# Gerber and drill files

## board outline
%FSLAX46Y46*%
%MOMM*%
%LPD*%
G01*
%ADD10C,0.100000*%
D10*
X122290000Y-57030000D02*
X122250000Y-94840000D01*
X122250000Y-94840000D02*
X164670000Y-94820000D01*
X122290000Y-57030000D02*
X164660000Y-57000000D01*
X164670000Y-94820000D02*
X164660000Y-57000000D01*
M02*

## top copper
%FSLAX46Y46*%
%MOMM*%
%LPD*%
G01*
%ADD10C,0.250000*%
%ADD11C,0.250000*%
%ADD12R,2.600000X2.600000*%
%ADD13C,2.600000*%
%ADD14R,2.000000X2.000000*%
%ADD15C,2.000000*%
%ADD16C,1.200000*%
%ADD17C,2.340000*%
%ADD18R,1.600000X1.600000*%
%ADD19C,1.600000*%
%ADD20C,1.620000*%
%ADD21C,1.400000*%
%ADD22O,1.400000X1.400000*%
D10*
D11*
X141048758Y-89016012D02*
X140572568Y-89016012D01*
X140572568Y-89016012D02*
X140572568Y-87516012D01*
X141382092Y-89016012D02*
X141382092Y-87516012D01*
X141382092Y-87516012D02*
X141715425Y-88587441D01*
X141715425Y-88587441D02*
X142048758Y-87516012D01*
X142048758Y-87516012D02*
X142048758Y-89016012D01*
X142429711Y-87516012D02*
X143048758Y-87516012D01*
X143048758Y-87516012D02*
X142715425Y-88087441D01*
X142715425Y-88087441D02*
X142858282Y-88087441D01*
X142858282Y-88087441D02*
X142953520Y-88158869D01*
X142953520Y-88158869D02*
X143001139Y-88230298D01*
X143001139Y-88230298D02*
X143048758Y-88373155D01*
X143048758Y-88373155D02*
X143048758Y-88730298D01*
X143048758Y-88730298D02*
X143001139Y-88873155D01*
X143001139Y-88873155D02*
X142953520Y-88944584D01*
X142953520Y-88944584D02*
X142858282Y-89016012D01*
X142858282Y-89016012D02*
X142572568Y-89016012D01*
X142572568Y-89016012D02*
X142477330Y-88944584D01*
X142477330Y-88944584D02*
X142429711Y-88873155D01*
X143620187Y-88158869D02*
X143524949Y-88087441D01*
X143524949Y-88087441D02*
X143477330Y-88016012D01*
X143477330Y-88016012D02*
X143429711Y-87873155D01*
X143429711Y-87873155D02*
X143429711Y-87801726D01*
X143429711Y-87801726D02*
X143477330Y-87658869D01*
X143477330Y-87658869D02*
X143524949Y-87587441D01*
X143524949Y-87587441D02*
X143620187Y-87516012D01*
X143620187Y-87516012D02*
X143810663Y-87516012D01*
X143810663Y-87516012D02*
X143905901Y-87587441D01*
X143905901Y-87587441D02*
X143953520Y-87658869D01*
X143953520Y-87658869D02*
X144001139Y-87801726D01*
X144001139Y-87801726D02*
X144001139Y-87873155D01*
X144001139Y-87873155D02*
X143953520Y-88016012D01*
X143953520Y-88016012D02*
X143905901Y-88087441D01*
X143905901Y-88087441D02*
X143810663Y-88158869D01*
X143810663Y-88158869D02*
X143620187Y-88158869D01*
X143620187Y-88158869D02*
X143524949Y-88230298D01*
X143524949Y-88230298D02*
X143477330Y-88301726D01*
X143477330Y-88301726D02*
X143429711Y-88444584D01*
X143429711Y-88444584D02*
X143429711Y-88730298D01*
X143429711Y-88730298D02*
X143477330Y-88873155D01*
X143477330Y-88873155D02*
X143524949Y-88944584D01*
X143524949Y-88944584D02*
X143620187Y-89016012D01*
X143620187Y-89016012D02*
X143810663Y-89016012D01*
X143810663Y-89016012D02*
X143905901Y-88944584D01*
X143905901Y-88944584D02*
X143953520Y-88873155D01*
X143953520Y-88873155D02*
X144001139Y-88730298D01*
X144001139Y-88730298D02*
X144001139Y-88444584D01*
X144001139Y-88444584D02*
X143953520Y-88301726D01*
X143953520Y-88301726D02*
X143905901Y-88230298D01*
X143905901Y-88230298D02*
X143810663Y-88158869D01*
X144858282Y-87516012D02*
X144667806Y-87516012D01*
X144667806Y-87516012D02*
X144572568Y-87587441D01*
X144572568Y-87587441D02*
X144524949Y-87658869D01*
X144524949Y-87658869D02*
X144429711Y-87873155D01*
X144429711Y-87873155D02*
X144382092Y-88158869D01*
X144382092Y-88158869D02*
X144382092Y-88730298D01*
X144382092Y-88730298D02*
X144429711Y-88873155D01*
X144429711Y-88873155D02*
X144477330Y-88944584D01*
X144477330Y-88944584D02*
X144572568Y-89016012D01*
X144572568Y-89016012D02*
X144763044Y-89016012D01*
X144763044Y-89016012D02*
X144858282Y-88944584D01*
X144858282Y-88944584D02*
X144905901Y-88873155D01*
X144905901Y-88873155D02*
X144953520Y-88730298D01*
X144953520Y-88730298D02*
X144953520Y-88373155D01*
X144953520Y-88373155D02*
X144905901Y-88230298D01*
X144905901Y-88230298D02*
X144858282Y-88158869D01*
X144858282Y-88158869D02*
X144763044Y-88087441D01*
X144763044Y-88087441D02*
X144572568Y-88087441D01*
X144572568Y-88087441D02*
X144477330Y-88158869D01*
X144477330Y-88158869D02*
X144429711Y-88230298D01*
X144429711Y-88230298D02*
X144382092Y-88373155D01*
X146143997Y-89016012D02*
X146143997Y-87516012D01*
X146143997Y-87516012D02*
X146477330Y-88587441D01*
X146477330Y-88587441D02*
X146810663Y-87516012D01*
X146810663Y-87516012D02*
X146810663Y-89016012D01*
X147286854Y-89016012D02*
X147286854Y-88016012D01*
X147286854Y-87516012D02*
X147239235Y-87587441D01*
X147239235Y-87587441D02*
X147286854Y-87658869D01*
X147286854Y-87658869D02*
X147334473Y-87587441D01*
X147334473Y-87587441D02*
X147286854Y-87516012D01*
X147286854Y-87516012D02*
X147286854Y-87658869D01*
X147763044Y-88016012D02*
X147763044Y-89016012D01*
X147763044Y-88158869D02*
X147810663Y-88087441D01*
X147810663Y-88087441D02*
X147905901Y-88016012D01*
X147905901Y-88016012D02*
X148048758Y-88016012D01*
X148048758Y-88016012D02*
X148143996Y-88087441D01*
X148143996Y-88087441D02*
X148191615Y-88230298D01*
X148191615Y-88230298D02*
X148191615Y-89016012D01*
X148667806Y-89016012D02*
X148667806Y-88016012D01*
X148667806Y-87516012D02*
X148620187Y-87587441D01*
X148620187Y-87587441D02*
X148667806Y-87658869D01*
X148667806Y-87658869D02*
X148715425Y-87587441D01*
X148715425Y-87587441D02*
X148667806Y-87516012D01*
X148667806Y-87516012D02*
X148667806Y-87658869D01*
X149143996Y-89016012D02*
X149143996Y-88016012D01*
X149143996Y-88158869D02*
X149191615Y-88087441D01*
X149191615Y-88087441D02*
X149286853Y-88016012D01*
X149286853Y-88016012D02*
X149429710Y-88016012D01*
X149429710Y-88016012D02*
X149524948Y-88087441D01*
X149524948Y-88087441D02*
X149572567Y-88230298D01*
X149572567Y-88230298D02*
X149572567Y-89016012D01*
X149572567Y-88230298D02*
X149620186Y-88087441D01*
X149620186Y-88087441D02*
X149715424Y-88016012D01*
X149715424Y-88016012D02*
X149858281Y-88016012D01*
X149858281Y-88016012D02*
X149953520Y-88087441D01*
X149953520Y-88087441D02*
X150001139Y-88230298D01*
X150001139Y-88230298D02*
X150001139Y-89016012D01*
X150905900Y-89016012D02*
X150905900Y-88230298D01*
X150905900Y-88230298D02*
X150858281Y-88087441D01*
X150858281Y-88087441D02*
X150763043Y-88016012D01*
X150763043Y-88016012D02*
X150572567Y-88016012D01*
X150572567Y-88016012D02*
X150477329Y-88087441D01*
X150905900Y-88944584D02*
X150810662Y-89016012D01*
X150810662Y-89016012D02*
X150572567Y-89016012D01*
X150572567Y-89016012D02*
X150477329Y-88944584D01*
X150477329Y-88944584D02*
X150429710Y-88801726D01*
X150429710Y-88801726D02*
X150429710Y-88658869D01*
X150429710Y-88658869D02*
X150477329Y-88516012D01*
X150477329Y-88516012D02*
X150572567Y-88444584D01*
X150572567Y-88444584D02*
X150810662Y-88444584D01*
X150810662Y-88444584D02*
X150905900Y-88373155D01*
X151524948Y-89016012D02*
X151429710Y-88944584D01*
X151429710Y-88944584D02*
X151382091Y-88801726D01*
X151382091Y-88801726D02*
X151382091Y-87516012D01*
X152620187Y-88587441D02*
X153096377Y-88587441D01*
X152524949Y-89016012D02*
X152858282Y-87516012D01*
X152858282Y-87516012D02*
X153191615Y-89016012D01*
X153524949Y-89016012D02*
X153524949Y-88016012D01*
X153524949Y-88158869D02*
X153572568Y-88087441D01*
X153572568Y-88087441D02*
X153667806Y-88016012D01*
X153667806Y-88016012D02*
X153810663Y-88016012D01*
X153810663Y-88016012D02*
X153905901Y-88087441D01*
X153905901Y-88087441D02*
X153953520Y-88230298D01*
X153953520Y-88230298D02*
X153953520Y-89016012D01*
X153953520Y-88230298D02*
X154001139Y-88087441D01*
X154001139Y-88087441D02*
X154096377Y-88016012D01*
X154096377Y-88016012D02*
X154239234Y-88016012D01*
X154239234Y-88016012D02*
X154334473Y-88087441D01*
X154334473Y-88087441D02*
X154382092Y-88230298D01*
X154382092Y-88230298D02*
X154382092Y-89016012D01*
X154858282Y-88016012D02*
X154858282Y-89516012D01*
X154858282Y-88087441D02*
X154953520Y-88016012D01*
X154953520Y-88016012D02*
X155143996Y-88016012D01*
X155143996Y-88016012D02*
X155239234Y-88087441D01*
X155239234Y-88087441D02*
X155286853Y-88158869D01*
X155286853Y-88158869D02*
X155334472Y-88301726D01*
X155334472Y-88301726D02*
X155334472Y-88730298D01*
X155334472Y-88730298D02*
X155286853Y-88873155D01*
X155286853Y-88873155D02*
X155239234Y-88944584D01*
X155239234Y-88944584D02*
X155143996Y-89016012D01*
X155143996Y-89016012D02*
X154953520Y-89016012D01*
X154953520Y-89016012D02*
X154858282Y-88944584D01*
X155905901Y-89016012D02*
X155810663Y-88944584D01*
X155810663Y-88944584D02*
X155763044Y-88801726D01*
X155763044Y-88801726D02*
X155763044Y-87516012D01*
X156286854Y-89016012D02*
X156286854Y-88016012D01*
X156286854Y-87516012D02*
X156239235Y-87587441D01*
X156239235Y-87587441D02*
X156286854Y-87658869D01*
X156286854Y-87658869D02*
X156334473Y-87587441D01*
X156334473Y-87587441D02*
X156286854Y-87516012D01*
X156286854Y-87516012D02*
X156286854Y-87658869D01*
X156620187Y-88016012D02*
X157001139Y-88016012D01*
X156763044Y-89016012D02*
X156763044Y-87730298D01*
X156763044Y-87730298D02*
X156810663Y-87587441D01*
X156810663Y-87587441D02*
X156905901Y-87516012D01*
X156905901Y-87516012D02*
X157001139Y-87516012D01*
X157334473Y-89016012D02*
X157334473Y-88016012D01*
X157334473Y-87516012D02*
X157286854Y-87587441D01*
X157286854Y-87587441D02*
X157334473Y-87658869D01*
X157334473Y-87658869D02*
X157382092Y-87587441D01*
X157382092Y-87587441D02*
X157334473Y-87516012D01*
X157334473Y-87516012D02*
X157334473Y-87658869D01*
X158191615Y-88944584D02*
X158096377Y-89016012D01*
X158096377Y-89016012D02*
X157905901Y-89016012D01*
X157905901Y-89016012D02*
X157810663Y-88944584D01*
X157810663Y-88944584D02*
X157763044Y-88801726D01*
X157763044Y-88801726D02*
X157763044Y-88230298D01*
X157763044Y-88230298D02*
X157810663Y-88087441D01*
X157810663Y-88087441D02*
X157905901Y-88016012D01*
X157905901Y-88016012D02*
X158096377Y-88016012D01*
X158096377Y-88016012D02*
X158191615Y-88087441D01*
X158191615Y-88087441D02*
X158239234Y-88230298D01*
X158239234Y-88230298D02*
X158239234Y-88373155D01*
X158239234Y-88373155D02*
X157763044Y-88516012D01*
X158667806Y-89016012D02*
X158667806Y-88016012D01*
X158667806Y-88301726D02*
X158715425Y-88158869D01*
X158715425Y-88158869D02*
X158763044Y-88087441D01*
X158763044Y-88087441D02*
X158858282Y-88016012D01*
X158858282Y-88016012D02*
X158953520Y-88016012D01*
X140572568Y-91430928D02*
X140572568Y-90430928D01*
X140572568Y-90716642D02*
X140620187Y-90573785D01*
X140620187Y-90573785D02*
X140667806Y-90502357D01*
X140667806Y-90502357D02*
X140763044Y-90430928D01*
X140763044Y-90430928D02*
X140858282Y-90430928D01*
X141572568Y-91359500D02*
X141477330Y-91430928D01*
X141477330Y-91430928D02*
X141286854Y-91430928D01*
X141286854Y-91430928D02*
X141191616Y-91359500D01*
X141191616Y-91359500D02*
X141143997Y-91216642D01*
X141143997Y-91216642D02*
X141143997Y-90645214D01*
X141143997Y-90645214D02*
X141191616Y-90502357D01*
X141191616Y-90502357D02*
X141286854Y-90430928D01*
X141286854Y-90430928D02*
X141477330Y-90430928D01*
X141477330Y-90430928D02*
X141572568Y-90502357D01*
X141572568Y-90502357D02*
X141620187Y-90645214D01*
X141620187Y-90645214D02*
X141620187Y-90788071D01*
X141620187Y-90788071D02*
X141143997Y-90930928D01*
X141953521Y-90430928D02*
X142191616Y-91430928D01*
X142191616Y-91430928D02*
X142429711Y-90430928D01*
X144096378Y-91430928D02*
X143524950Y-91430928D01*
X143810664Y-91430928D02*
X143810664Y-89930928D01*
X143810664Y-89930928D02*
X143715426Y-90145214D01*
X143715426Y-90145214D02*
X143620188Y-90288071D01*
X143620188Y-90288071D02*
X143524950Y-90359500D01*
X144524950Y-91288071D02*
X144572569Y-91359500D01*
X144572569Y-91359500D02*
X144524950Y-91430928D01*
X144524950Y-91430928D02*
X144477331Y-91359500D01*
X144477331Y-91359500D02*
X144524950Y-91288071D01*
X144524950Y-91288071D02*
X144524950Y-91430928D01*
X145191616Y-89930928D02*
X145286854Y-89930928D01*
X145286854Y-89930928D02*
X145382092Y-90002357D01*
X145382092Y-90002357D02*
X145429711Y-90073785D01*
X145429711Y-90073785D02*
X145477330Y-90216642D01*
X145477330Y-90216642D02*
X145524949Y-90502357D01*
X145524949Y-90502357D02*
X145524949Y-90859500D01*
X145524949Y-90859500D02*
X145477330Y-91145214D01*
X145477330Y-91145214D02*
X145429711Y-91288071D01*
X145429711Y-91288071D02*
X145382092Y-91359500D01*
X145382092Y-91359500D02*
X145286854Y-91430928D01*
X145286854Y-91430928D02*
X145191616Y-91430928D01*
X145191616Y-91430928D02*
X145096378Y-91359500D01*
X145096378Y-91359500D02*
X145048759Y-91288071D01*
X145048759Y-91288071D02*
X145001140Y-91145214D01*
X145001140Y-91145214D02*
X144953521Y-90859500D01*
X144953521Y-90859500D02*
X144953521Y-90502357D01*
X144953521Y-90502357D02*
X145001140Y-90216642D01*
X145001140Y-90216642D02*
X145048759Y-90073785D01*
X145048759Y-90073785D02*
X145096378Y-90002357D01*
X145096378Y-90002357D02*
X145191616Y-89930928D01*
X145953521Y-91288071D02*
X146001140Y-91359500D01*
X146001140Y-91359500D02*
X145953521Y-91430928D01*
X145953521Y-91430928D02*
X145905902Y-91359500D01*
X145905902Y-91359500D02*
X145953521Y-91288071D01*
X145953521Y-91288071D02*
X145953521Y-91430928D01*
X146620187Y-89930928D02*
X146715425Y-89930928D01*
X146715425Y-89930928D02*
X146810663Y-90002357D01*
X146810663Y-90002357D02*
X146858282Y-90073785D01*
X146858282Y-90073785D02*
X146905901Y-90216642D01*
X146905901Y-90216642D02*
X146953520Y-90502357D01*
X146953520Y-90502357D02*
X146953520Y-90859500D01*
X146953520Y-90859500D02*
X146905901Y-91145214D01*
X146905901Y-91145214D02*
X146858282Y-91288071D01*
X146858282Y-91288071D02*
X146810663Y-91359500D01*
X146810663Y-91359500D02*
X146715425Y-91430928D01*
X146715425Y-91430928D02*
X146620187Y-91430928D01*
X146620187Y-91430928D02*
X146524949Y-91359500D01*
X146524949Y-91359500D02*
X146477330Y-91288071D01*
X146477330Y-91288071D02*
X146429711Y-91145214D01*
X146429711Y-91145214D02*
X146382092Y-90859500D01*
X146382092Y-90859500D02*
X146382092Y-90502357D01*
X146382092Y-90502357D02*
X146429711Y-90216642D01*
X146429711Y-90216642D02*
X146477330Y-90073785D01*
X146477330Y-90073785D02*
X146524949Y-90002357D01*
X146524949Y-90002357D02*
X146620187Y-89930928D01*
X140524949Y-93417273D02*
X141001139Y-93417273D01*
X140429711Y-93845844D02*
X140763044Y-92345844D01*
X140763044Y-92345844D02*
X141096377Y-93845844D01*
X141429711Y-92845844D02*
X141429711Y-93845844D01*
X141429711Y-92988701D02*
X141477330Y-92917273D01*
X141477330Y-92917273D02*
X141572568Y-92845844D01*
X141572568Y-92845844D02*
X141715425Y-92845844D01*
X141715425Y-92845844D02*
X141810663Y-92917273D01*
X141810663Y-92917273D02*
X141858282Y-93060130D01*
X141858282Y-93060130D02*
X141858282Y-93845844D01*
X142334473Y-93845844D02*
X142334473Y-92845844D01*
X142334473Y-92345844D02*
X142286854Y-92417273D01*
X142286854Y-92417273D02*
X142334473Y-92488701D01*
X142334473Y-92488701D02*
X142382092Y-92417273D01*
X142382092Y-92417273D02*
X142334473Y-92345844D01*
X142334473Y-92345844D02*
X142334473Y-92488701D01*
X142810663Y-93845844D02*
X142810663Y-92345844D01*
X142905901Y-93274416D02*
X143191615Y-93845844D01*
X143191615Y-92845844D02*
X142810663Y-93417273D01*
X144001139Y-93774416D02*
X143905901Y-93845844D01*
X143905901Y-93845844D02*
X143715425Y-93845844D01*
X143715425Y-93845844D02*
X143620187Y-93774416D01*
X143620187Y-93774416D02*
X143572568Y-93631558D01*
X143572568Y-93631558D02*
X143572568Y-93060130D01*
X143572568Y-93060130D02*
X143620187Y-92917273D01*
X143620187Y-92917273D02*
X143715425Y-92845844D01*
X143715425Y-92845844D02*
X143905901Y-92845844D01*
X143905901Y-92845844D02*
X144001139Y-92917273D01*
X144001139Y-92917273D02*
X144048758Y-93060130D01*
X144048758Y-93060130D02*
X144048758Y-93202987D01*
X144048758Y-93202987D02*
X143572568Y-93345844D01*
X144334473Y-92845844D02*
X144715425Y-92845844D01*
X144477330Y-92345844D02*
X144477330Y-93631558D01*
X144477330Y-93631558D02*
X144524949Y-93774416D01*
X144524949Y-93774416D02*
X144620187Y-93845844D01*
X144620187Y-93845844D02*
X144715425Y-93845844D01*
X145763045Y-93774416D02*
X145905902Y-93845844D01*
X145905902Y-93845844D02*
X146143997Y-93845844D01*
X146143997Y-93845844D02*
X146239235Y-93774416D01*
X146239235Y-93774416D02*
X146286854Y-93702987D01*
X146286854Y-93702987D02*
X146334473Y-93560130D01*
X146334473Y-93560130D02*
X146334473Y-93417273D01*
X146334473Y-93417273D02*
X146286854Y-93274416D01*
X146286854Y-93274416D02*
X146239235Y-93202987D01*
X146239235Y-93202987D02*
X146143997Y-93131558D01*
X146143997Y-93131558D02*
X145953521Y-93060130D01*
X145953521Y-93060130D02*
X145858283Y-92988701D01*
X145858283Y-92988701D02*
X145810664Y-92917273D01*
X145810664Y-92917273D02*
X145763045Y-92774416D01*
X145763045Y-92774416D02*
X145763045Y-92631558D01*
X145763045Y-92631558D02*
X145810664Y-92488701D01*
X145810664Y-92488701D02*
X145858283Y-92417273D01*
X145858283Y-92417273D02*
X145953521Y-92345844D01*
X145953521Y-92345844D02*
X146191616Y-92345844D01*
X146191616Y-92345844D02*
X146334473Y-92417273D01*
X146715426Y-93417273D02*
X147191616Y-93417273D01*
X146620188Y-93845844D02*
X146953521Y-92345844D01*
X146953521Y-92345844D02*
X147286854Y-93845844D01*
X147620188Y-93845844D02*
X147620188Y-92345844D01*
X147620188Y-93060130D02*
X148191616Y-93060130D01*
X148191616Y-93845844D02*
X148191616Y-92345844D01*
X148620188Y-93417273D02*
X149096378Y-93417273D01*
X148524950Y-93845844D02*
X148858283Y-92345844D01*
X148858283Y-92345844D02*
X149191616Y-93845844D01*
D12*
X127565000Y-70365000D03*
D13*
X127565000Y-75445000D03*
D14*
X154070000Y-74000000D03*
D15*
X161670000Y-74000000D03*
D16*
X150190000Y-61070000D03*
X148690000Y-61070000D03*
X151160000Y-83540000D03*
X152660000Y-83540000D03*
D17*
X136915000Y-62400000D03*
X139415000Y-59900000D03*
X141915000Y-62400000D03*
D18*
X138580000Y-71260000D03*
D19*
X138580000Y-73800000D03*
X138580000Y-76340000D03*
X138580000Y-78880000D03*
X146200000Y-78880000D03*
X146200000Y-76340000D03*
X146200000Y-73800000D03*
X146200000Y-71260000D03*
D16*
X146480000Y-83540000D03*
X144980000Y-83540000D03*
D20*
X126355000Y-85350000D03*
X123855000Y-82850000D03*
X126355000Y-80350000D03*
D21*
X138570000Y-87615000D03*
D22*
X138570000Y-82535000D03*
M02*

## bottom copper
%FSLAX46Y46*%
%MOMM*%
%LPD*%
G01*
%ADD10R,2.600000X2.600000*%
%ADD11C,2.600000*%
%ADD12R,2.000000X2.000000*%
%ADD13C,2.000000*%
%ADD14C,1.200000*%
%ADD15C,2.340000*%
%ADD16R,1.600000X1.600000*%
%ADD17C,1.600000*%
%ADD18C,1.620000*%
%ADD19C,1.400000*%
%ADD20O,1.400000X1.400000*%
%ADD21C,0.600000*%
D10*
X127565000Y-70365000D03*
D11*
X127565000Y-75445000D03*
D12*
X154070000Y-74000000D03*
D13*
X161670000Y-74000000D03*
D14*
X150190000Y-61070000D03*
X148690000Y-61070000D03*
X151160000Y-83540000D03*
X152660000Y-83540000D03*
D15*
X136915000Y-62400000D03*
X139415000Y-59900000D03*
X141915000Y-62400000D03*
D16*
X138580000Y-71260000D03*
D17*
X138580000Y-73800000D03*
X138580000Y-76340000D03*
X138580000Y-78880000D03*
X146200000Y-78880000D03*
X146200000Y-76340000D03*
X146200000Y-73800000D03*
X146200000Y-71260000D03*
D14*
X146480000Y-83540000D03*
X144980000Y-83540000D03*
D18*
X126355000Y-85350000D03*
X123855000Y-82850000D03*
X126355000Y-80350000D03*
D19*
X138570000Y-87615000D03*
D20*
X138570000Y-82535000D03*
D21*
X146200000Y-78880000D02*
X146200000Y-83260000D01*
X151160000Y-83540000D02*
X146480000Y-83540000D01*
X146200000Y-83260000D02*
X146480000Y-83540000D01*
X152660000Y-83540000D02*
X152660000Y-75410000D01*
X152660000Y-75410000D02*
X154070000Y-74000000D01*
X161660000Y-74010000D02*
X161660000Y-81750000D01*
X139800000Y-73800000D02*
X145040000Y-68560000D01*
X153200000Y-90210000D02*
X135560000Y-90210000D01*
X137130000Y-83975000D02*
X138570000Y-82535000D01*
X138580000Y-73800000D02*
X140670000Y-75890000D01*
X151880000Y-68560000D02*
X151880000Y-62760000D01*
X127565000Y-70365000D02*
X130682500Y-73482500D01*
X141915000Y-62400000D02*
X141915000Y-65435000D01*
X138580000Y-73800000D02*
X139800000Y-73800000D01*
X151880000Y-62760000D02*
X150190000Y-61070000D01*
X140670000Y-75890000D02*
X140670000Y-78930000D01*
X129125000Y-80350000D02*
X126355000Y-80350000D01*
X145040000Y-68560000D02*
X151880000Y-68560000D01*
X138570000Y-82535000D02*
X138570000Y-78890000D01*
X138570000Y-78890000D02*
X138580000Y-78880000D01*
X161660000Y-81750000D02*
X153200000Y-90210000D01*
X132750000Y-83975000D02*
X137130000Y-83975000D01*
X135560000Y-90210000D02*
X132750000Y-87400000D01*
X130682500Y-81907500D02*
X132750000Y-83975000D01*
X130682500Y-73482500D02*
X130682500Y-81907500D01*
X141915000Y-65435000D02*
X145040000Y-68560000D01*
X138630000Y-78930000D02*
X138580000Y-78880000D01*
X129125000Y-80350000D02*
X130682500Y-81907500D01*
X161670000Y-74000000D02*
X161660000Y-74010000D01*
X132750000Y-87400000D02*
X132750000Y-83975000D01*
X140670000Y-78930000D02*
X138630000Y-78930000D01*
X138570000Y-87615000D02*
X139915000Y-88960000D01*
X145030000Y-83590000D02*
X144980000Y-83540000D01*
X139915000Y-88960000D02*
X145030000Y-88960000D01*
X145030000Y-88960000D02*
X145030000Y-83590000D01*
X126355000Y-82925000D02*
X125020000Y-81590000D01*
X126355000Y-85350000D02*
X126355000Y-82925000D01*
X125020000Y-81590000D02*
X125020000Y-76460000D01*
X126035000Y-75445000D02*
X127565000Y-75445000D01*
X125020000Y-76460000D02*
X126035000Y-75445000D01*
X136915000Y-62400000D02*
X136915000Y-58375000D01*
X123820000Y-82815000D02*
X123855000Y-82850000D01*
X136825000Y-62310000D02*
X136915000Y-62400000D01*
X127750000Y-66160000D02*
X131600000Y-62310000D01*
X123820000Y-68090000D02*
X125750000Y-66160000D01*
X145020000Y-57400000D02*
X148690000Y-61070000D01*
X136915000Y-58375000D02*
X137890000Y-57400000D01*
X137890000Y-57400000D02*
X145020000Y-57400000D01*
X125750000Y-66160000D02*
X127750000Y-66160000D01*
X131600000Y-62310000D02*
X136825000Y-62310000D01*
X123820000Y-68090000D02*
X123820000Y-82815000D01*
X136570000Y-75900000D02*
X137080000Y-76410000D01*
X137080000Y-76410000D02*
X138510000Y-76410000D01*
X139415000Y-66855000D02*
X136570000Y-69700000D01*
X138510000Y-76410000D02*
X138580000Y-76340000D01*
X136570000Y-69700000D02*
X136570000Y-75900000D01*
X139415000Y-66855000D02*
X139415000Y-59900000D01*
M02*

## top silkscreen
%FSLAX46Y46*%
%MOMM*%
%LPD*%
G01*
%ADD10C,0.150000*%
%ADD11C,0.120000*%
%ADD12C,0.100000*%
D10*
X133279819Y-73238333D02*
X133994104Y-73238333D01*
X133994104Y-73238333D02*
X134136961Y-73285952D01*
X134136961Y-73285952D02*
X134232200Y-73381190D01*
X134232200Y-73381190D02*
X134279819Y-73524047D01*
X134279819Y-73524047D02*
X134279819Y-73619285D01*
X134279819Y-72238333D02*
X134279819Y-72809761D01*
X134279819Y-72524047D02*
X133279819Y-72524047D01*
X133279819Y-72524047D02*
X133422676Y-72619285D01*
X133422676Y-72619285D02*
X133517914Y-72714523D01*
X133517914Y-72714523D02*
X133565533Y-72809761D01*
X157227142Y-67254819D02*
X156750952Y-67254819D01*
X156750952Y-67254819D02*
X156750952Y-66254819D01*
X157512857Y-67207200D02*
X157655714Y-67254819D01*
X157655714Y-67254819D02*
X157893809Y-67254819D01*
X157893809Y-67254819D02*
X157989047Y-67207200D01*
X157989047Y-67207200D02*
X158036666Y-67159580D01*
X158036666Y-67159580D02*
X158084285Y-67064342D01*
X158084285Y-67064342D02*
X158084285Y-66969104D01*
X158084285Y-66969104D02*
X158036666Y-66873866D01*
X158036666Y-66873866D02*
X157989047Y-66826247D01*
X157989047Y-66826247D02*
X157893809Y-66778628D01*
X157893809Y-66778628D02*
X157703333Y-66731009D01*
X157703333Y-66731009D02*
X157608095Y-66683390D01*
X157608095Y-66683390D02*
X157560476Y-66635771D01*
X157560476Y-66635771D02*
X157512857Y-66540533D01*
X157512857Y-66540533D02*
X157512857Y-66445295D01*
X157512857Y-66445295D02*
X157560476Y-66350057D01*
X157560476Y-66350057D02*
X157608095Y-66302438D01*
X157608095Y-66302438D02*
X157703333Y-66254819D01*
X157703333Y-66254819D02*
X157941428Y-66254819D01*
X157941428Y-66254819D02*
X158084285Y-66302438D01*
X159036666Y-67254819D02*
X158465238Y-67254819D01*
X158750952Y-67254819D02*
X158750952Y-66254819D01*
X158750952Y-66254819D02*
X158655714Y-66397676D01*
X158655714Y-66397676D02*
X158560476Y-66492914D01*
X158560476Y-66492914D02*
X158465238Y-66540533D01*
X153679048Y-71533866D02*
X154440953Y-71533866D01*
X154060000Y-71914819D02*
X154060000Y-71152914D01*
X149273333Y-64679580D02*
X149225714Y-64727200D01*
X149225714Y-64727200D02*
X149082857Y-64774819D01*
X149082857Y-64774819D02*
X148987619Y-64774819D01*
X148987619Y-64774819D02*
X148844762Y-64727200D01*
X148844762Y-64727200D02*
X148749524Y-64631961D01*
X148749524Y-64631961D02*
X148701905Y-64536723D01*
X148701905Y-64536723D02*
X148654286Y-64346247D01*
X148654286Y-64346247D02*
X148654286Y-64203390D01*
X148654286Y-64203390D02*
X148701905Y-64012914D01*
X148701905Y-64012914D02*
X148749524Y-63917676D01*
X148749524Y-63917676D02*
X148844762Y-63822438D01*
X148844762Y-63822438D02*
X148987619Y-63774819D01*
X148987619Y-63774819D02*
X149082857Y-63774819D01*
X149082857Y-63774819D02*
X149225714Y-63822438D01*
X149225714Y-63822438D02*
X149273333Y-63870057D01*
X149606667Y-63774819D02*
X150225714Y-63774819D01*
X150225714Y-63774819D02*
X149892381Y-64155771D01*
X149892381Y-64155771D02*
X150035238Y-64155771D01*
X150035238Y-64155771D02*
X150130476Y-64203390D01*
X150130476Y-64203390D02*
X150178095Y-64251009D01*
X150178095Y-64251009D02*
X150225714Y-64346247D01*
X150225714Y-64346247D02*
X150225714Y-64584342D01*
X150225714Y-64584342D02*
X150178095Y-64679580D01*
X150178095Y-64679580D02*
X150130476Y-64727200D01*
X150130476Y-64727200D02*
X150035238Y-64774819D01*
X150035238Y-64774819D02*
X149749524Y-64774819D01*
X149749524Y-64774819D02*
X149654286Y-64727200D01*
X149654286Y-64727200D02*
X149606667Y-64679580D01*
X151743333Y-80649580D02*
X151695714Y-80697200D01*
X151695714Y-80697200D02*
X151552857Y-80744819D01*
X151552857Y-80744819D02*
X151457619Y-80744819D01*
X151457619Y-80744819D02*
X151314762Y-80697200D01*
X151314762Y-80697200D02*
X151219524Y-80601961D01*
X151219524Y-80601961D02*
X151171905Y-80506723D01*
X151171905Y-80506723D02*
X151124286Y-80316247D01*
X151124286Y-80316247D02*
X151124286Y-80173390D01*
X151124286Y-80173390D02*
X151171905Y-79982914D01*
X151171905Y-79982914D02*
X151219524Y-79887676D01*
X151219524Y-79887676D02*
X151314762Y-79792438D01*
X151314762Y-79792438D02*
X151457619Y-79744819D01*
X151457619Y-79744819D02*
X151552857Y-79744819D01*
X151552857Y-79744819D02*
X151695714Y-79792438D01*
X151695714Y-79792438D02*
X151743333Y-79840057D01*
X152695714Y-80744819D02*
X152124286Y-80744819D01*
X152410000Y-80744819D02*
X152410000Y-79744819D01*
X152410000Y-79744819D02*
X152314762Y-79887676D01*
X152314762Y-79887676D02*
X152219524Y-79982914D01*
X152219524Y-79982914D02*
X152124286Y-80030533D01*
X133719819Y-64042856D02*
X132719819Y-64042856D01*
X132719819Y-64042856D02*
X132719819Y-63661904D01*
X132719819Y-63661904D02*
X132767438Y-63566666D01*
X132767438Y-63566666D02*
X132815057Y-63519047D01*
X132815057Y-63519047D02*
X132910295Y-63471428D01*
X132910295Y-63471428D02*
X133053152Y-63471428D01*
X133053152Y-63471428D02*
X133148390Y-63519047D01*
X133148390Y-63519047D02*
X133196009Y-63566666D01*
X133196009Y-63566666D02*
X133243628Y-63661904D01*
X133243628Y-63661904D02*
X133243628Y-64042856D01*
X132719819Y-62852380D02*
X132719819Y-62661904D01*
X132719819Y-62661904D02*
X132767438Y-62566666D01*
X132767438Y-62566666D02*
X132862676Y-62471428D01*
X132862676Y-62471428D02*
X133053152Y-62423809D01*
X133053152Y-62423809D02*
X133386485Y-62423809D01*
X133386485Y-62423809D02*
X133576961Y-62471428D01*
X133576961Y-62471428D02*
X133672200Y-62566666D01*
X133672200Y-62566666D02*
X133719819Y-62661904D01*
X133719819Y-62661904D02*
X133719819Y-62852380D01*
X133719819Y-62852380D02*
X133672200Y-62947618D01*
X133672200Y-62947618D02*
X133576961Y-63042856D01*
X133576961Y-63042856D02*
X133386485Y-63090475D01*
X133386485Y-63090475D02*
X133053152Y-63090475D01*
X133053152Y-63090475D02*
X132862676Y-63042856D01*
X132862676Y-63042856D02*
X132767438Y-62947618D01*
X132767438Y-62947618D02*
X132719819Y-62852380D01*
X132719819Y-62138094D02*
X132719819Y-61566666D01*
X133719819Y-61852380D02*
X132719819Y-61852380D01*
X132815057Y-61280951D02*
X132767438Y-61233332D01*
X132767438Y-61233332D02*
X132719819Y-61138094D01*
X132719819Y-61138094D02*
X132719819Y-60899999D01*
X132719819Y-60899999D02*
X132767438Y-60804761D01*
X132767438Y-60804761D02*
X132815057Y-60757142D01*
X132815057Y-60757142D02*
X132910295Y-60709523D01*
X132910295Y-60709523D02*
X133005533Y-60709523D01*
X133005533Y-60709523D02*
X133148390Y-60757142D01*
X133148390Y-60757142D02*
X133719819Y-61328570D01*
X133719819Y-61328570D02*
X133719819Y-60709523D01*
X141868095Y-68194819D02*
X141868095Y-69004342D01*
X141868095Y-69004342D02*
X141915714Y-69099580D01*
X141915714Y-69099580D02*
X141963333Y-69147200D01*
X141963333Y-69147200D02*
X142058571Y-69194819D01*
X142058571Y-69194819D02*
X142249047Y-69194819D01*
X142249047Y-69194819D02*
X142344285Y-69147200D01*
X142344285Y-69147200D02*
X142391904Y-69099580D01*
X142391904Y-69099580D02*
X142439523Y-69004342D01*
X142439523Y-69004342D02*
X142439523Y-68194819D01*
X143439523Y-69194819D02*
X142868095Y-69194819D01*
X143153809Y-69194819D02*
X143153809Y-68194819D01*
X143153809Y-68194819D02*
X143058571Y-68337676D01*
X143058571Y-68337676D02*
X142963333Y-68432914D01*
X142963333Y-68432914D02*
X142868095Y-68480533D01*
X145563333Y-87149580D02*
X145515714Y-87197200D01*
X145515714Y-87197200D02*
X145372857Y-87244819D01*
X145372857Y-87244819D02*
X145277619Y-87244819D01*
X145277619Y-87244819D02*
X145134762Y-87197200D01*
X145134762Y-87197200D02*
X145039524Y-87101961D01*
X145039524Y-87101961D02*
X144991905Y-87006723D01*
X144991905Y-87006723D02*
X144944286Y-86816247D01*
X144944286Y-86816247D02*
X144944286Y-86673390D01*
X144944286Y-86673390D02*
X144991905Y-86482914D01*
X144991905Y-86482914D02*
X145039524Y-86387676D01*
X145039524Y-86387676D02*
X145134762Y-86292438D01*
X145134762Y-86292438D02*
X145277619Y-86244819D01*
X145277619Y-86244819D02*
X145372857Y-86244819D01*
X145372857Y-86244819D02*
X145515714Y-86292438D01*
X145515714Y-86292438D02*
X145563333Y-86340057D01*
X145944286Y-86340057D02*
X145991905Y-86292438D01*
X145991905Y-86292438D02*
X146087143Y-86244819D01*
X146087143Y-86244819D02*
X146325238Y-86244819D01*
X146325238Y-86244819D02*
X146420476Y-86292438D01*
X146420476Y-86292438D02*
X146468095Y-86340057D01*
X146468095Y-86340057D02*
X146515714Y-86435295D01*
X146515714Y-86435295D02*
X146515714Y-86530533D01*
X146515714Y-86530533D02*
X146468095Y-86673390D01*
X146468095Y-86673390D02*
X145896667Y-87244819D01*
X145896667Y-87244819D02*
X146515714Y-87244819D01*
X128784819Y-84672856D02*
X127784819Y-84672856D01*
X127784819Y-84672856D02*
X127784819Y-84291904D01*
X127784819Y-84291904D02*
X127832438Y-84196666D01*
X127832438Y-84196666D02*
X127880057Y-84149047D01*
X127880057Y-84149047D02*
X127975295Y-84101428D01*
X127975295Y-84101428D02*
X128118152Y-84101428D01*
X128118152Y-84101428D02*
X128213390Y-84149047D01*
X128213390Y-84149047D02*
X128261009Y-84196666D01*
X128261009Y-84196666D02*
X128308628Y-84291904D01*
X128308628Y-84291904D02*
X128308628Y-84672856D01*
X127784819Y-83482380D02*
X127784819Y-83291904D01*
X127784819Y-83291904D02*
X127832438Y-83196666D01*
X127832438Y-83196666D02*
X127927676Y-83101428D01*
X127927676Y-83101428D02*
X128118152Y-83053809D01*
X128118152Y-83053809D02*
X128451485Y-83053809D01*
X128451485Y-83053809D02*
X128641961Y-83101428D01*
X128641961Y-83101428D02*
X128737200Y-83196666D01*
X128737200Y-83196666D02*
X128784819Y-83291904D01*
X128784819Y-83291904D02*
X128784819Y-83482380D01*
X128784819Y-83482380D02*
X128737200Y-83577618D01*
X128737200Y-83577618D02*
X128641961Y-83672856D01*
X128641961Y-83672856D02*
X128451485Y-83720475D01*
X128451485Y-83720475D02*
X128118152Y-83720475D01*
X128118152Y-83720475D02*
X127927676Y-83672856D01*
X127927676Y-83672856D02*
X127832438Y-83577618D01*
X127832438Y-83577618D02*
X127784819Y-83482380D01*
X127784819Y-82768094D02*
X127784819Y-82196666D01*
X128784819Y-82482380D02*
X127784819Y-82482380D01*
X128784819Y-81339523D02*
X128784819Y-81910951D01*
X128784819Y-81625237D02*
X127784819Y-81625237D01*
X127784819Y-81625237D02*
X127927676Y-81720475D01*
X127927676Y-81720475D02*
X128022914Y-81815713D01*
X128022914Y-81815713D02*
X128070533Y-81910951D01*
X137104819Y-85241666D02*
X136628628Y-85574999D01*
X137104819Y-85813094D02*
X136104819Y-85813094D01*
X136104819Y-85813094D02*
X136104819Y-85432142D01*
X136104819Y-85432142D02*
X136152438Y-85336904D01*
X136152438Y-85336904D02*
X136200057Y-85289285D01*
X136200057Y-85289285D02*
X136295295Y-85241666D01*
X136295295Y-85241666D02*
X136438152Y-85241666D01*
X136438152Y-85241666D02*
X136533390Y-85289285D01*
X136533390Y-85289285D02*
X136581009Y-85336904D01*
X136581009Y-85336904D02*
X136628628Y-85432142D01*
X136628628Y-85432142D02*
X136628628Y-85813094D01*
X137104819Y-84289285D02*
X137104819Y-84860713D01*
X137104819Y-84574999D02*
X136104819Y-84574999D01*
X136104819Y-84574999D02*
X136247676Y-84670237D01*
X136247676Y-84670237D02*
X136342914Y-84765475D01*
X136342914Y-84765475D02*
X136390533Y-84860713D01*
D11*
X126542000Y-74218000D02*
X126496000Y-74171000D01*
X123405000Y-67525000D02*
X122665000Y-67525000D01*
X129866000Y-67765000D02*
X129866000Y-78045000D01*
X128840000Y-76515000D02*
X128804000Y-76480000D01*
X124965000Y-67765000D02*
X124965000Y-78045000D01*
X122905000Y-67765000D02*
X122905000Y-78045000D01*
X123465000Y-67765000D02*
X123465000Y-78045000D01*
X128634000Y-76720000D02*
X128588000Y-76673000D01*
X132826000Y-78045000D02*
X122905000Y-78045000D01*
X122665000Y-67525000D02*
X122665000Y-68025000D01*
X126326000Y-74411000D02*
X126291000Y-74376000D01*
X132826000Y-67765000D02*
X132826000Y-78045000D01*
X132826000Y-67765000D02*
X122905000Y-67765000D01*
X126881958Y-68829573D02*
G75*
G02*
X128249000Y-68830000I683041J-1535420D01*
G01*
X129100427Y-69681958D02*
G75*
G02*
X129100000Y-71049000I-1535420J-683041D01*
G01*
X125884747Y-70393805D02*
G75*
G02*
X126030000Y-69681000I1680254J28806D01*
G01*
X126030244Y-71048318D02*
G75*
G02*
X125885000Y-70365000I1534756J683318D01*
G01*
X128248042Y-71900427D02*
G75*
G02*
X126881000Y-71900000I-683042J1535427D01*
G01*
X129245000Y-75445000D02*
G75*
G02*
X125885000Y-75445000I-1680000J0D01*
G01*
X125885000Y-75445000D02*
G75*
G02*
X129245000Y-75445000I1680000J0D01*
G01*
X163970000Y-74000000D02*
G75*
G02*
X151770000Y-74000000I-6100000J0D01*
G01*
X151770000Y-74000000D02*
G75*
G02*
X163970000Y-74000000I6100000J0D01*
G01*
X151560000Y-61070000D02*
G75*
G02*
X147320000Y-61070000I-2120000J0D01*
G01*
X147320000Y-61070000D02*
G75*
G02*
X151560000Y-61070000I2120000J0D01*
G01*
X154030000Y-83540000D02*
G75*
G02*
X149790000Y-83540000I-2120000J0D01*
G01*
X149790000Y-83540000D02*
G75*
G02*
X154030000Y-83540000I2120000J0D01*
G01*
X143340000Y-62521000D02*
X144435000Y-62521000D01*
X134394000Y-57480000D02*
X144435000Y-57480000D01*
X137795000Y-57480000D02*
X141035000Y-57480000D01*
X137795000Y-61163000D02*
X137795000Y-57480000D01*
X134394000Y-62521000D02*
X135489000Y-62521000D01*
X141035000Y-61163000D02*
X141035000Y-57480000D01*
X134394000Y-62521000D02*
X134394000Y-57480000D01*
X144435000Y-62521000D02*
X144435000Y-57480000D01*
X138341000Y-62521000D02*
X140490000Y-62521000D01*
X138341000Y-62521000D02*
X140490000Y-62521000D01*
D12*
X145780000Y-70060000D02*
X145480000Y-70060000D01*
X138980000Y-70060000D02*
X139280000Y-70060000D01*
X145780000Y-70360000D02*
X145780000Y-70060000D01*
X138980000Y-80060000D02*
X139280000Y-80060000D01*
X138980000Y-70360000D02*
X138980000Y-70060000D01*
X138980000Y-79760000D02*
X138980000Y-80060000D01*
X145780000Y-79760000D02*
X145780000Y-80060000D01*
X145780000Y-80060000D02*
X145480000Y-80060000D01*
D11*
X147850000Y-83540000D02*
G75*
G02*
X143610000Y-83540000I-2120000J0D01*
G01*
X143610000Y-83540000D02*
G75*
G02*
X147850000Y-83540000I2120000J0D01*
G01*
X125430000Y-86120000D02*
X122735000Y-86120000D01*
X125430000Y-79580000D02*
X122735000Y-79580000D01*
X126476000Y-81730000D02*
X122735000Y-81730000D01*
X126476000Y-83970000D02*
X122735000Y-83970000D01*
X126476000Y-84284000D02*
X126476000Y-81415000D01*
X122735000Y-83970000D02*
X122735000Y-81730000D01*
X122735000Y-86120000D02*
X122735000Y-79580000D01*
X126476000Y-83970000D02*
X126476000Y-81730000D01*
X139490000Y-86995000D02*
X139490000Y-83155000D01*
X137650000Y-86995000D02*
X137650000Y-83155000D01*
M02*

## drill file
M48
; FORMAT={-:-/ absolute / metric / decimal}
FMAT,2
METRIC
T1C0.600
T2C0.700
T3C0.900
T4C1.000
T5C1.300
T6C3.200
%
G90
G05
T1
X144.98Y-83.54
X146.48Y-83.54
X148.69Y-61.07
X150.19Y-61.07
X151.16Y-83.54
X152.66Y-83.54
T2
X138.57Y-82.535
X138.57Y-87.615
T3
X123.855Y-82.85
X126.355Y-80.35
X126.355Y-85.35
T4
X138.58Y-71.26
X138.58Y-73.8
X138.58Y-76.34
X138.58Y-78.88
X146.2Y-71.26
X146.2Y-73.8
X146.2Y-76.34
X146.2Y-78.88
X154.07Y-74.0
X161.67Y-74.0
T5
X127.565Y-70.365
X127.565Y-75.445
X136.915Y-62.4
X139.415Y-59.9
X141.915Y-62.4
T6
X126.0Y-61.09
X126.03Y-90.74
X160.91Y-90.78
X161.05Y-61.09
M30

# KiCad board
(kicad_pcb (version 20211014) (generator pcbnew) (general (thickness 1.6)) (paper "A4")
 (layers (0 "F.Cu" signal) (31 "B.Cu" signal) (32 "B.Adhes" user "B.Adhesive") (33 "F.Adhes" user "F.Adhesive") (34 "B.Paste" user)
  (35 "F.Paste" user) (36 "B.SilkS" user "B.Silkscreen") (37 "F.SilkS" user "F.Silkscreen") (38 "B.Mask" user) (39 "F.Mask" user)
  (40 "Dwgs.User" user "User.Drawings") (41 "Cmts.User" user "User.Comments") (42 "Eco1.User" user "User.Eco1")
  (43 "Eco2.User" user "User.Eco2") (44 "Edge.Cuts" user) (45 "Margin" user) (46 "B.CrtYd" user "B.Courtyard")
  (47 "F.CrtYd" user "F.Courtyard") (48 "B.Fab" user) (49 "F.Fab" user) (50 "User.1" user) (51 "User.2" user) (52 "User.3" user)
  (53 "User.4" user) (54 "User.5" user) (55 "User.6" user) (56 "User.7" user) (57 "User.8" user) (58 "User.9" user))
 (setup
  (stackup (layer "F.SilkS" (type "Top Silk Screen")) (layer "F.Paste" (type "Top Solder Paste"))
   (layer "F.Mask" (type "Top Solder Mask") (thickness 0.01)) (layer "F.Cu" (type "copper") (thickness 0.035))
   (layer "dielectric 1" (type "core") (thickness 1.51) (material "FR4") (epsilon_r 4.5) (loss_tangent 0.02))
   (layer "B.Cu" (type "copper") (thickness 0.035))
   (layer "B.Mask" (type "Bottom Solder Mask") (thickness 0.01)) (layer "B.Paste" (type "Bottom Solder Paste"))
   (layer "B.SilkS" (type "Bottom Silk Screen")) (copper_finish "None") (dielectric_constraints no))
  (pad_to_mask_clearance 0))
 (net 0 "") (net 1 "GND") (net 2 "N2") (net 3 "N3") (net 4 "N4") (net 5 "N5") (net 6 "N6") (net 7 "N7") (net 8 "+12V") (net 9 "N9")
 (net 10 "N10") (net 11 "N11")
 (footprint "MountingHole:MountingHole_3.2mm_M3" (layer "F.Cu") (at 126.03 90.74)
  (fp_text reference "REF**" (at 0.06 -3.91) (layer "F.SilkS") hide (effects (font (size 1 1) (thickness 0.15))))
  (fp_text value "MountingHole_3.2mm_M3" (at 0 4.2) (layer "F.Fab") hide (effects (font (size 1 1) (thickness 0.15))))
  (pad "" np_thru_hole circle (at 0 0) (size 3.2 3.2) (drill 3.2) (layers *.Cu *.Mask)))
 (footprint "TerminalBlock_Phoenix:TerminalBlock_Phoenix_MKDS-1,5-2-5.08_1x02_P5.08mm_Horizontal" (layer "F.Cu") (at 127.565 70.365 -90)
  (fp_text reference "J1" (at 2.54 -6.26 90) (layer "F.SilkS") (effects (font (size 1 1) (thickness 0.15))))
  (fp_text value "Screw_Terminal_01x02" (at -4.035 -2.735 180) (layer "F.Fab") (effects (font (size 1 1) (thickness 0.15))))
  (fp_line (start 3.853 1.023) (end 3.806 1.069) (layer "F.SilkS") (width 0.12))
  (fp_line (start -2.84 4.16) (end -2.84 4.9) (layer "F.SilkS") (width 0.12))
  (fp_line (start -2.6 -2.301) (end 7.68 -2.301) (layer "F.SilkS") (width 0.12))
  (fp_line (start 6.15 -1.275) (end 6.115 -1.239) (layer "F.SilkS") (width 0.12))
  (fp_line (start -2.6 2.6) (end 7.68 2.6) (layer "F.SilkS") (width 0.12))
  (fp_line (start -2.6 4.66) (end 7.68 4.66) (layer "F.SilkS") (width 0.12))
  (fp_line (start -2.6 4.1) (end 7.68 4.1) (layer "F.SilkS") (width 0.12))
  (fp_line (start 6.355 -1.069) (end 6.308 -1.023) (layer "F.SilkS") (width 0.12))
  (fp_line (start 7.68 -5.261) (end 7.68 4.66) (layer "F.SilkS") (width 0.12))
  (fp_line (start -2.84 4.9) (end -2.34 4.9) (layer "F.SilkS") (width 0.12))
  (fp_line (start 4.046 1.239) (end 4.011 1.274) (layer "F.SilkS") (width 0.12))
  (fp_line (start -2.6 -5.261) (end 7.68 -5.261) (layer "F.SilkS") (width 0.12))
  (fp_line (start -2.6 -5.261) (end -2.6 4.66) (layer "F.SilkS") (width 0.12))
  (fp_arc (start -1.535427 0.683042) (mid -1.680501 -0.000524) (end -1.535 -0.684) (layer "F.SilkS") (width 0.12))
  (fp_arc (start -0.683042 -1.535427) (mid 0.000524 -1.680501) (end 0.684 -1.535) (layer "F.SilkS") (width 0.12))
  (fp_arc (start 0.028805 1.680253) (mid -0.335551 1.646659) (end -0.684 1.535) (layer "F.SilkS") (width 0.12))
  (fp_arc (start 0.683318 1.534756) (mid 0.349292 1.643288) (end 0 1.68) (layer "F.SilkS") (width 0.12))
  (fp_arc (start 1.535427 -0.683042) (mid 1.680501 0.000524) (end 1.535 0.684) (layer "F.SilkS") (width 0.12))
  (fp_circle (center 5.08 0) (end 6.76 0) (layer "F.SilkS") (width 0.12) (fill none))
  (pad "1" thru_hole rect (at 0 0 270) (size 2.6 2.6) (drill 1.3) (layers *.Cu *.Mask) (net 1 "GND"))
  (pad "2" thru_hole circle (at 5.08 0 270) (size 2.6 2.6) (drill 1.3) (layers *.Cu *.Mask) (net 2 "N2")))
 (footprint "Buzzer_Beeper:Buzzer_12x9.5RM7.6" (layer "F.Cu") (at 154.07 74)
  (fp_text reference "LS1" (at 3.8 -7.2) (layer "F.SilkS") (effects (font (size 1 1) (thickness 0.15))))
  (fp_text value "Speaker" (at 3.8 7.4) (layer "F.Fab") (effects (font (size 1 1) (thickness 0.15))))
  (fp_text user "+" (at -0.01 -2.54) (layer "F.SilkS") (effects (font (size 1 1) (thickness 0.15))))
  (fp_circle (center 3.8 0) (end 9.9 0) (layer "F.SilkS") (width 0.12) (fill none))
  (pad "1" thru_hole rect (at 0 0) (size 2 2) (drill 1) (layers *.Cu *.Mask) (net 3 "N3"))
  (pad "2" thru_hole circle (at 7.6 0) (size 2 2) (drill 1) (layers *.Cu *.Mask) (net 1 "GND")))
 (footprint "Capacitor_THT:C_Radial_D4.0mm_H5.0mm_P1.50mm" (layer "F.Cu") (at 150.19 61.07 180)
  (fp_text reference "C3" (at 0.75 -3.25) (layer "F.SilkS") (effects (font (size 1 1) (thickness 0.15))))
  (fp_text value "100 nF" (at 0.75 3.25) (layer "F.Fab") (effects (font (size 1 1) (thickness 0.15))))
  (fp_circle (center 0.75 0) (end 2.87 0) (layer "F.SilkS") (width 0.12) (fill none))
  (pad "1" thru_hole circle (at 0 0 180) (size 1.2 1.2) (drill 0.6) (layers *.Cu *.Mask) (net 1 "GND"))
  (pad "2" thru_hole circle (at 1.5 0 180) (size 1.2 1.2) (drill 0.6) (layers *.Cu *.Mask) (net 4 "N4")))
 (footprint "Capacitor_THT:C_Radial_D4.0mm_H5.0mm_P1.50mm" (layer "F.Cu") (at 151.16 83.54)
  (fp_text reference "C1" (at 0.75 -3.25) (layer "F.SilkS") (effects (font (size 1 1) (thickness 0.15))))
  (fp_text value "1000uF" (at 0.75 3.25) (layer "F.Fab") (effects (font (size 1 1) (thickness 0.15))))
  (fp_circle (center 0.75 0) (end 2.87 0) (layer "F.SilkS") (width 0.12) (fill none))
  (pad "1" thru_hole circle (at 0 0) (size 1.2 1.2) (drill 0.6) (layers *.Cu *.Mask) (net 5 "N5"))
  (pad "2" thru_hole circle (at 1.5 0) (size 1.2 1.2) (drill 0.6) (layers *.Cu *.Mask) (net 3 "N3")))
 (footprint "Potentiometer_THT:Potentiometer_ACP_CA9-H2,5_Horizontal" (layer "F.Cu") (at 136.915 62.4 90)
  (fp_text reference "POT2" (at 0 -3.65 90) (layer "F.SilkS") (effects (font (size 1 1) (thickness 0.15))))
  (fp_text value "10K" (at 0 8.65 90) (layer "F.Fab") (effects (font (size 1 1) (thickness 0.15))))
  (fp_line (start -0.121 6.425) (end -0.121 7.52) (layer "F.SilkS") (width 0.12))
  (fp_line (start 4.92 -2.521) (end 4.92 7.52) (layer "F.SilkS") (width 0.12))
  (fp_line (start 4.92 0.88) (end 4.92 4.12) (layer "F.SilkS") (width 0.12))
  (fp_line (start 1.237 0.88) (end 4.92 0.88) (layer "F.SilkS") (width 0.12))
  (fp_line (start -0.121 -2.521) (end -0.121 -1.426) (layer "F.SilkS") (width 0.12))
  (fp_line (start 1.237 4.12) (end 4.92 4.12) (layer "F.SilkS") (width 0.12))
  (fp_line (start -0.121 -2.521) (end 4.92 -2.521) (layer "F.SilkS") (width 0.12))
  (fp_line (start -0.121 7.52) (end 4.92 7.52) (layer "F.SilkS") (width 0.12))
  (fp_line (start -0.121 1.426) (end -0.121 3.575) (layer "F.SilkS") (width 0.12))
  (fp_line (start -0.121 1.426) (end -0.121 3.575) (layer "F.SilkS") (width 0.12))
  (pad "1" thru_hole circle (at 0 0 90) (size 2.34 2.34) (drill 1.3) (layers *.Cu *.Mask) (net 4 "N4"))
  (pad "2" thru_hole circle (at 2.5 2.5 90) (size 2.34 2.34) (drill 1.3) (layers *.Cu *.Mask) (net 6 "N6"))
  (pad "3" thru_hole circle (at 0 5 90) (size 2.34 2.34) (drill 1.3) (layers *.Cu *.Mask) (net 1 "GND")))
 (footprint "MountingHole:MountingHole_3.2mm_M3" (layer "F.Cu") (at 160.91 90.78)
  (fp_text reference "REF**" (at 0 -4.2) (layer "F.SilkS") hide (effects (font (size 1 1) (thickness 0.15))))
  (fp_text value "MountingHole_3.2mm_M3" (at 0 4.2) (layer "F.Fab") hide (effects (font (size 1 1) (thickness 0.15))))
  (pad "" np_thru_hole circle (at 0 0) (size 3.2 3.2) (drill 3.2) (layers *.Cu *.Mask)))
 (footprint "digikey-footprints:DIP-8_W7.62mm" (layer "F.Cu") (at 138.58 71.26)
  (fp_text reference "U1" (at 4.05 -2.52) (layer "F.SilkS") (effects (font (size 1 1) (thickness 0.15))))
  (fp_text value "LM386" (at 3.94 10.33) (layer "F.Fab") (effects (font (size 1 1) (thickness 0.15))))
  (fp_line (start 7.2 -1.2) (end 6.9 -1.2) (layer "F.SilkS") (width 0.1))
  (fp_line (start 0.4 -1.2) (end 0.7 -1.2) (layer "F.SilkS") (width 0.1))
  (fp_line (start 7.2 -0.9) (end 7.2 -1.2) (layer "F.SilkS") (width 0.1))
  (fp_line (start 0.4 8.8) (end 0.7 8.8) (layer "F.SilkS") (width 0.1))
  (fp_line (start 0.4 -0.9) (end 0.4 -1.2) (layer "F.SilkS") (width 0.1))
  (fp_line (start 0.4 8.5) (end 0.4 8.8) (layer "F.SilkS") (width 0.1))
  (fp_line (start 7.2 8.5) (end 7.2 8.8) (layer "F.SilkS") (width 0.1))
  (fp_line (start 7.2 8.8) (end 6.9 8.8) (layer "F.SilkS") (width 0.1))
  (pad "1" thru_hole rect locked (at 0 0) (size 1.6 1.6) (drill 1) (layers *.Cu *.Mask) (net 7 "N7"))
  (pad "2" thru_hole circle locked (at 0 2.54) (size 1.6 1.6) (drill 1) (layers *.Cu *.Mask) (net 1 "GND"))
  (pad "3" thru_hole circle locked (at 0 5.08) (size 1.6 1.6) (drill 1) (layers *.Cu *.Mask) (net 6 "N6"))
  (pad "4" thru_hole circle locked (at 0 7.62) (size 1.6 1.6) (drill 1) (layers *.Cu *.Mask) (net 1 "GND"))
  (pad "5" thru_hole circle locked (at 7.62 7.62) (size 1.6 1.6) (drill 1) (layers *.Cu *.Mask) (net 5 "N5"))
  (pad "6" thru_hole circle locked (at 7.62 5.08) (size 1.6 1.6) (drill 1) (layers *.Cu *.Mask) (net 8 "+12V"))
  (pad "7" thru_hole circle locked (at 7.62 2.54) (size 1.6 1.6) (drill 1) (layers *.Cu *.Mask) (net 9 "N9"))
  (pad "8" thru_hole circle locked (at 7.62 0) (size 1.6 1.6) (drill 1) (layers *.Cu *.Mask) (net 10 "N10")))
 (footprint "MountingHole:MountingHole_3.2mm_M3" (layer "F.Cu") (at 126 61.09)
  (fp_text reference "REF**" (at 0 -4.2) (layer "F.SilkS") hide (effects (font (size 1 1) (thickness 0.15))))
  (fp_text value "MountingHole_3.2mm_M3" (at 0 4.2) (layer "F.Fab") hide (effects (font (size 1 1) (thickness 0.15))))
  (pad "" np_thru_hole circle (at 0 0) (size 3.2 3.2) (drill 3.2) (layers *.Cu *.Mask)))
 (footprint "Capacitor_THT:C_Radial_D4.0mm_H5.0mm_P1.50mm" (layer "F.Cu") (at 146.48 83.54 180)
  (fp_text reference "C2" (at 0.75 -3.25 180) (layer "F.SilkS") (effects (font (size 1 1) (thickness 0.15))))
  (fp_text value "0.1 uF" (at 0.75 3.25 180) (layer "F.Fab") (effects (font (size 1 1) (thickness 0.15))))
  (fp_circle (center 0.75 0) (end 2.87 0) (layer "F.SilkS") (width 0.12) (fill none))
  (pad "1" thru_hole circle (at 0 0 180) (size 1.2 1.2) (drill 0.6) (layers *.Cu *.Mask) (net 5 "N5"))
  (pad "2" thru_hole circle (at 1.5 0 180) (size 1.2 1.2) (drill 0.6) (layers *.Cu *.Mask) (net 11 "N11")))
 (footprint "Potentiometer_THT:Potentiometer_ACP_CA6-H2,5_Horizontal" (layer "F.Cu") (at 126.355 85.35 180)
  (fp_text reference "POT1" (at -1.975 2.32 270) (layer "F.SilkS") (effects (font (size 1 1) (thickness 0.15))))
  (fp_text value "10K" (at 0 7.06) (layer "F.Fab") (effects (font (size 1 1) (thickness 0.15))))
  (fp_line (start 0.925 -0.77) (end 3.62 -0.77) (layer "F.SilkS") (width 0.12))
  (fp_line (start 0.925 5.77) (end 3.62 5.77) (layer "F.SilkS") (width 0.12))
  (fp_line (start -0.121 3.62) (end 3.62 3.62) (layer "F.SilkS") (width 0.12))
  (fp_line (start -0.121 1.38) (end 3.62 1.38) (layer "F.SilkS") (width 0.12))
  (fp_line (start -0.121 1.066) (end -0.121 3.935) (layer "F.SilkS") (width 0.12))
  (fp_line (start 3.62 1.38) (end 3.62 3.62) (layer "F.SilkS") (width 0.12))
  (fp_line (start 3.62 -0.77) (end 3.62 5.77) (layer "F.SilkS") (width 0.12))
  (fp_line (start -0.121 1.38) (end -0.121 3.62) (layer "F.SilkS") (width 0.12))
  (pad "1" thru_hole circle (at 0 0 180) (size 1.62 1.62) (drill 0.9) (layers *.Cu *.Mask) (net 2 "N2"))
  (pad "2" thru_hole circle (at 2.5 2.5 180) (size 1.62 1.62) (drill 0.9) (layers *.Cu *.Mask) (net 4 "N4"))
  (pad "3" thru_hole circle (at 0 5 180) (size 1.62 1.62) (drill 0.9) (layers *.Cu *.Mask) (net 1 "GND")))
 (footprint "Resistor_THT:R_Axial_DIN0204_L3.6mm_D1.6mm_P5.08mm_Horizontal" (layer "F.Cu") (at 138.57 87.615 90)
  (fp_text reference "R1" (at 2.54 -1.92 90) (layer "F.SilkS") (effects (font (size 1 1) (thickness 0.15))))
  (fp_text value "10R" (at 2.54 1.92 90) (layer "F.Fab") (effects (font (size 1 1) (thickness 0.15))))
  (fp_line (start 0.62 0.92) (end 4.46 0.92) (layer "F.SilkS") (width 0.12))
  (fp_line (start 0.62 -0.92) (end 4.46 -0.92) (layer "F.SilkS") (width 0.12))
  (pad "1" thru_hole circle (at 0 0 90) (size 1.4 1.4) (drill 0.7) (layers *.Cu *.Mask) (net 11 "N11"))
  (pad "2" thru_hole oval (at 5.08 0 90) (size 1.4 1.4) (drill 0.7) (layers *.Cu *.Mask) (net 1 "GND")))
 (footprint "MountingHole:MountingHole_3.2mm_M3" (layer "F.Cu") (at 161.05 61.09)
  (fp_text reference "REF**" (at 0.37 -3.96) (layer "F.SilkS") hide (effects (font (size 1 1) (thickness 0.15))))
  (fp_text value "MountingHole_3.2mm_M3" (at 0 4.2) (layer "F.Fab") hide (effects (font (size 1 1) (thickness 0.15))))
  (pad "" np_thru_hole circle (at 0 0) (size 3.2 3.2) (drill 3.2) (layers *.Cu *.Mask)))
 (gr_line (start 122.29 57.03) (end 122.25 94.84) (layer "Edge.Cuts") (width 0.1))
 (gr_line (start 122.25 94.84) (end 164.67 94.82) (layer "Edge.Cuts") (width 0.1))
 (gr_line (start 122.29 57.03) (end 164.66 57) (layer "Edge.Cuts") (width 0.1))
 (gr_line (start 164.67 94.82) (end 164.66 57) (layer "Edge.Cuts") (width 0.1))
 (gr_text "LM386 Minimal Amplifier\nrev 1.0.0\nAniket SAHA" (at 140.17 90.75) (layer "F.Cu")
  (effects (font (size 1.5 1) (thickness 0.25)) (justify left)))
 (segment (start 146.2 78.88) (end 146.2 83.26) (width 0.6) (layer "B.Cu") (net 5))
 (segment (start 151.16 83.54) (end 146.48 83.54) (width 0.6) (layer "B.Cu") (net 5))
 (segment (start 146.2 83.26) (end 146.48 83.54) (width 0.6) (layer "B.Cu") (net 5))
 (segment (start 152.66 83.54) (end 152.66 75.41) (width 0.6) (layer "B.Cu") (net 3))
 (segment (start 152.66 75.41) (end 154.07 74) (width 0.6) (layer "B.Cu") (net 3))
 (segment (start 161.66 74.01) (end 161.66 81.75) (width 0.6) (layer "B.Cu") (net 1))
 (segment (start 139.8 73.8) (end 145.04 68.56) (width 0.6) (layer "B.Cu") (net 1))
 (segment (start 153.2 90.21) (end 135.56 90.21) (width 0.6) (layer "B.Cu") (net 1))
 (segment (start 137.13 83.975) (end 138.57 82.535) (width 0.6) (layer "B.Cu") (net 1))
 (segment (start 138.58 73.8) (end 140.67 75.89) (width 0.6) (layer "B.Cu") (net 1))
 (segment (start 151.88 68.56) (end 151.88 62.76) (width 0.6) (layer "B.Cu") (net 1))
 (segment (start 127.565 70.365) (end 130.6825 73.4825) (width 0.6) (layer "B.Cu") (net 1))
 (segment (start 141.915 62.4) (end 141.915 65.435) (width 0.6) (layer "B.Cu") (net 1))
 (segment (start 138.58 73.8) (end 139.8 73.8) (width 0.6) (layer "B.Cu") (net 1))
 (segment (start 151.88 62.76) (end 150.19 61.07) (width 0.6) (layer "B.Cu") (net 1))
 (segment (start 140.67 75.89) (end 140.67 78.93) (width 0.6) (layer "B.Cu") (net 1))
 (segment (start 129.125 80.35) (end 126.355 80.35) (width 0.6) (layer "B.Cu") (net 1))
 (segment (start 145.04 68.56) (end 151.88 68.56) (width 0.6) (layer "B.Cu") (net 1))
 (segment (start 138.57 82.535) (end 138.57 78.89) (width 0.6) (layer "B.Cu") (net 1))
 (segment (start 138.57 78.89) (end 138.58 78.88) (width 0.6) (layer "B.Cu") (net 1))
 (segment (start 161.66 81.75) (end 153.2 90.21) (width 0.6) (layer "B.Cu") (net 1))
 (segment (start 132.75 83.975) (end 137.13 83.975) (width 0.6) (layer "B.Cu") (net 1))
 (segment (start 135.56 90.21) (end 132.75 87.4) (width 0.6) (layer "B.Cu") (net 1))
 (segment (start 130.6825 81.9075) (end 132.75 83.975) (width 0.6) (layer "B.Cu") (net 1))
 (segment (start 130.6825 73.4825) (end 130.6825 81.9075) (width 0.6) (layer "B.Cu") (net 1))
 (segment (start 141.915 65.435) (end 145.04 68.56) (width 0.6) (layer "B.Cu") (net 1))
 (segment (start 138.63 78.93) (end 138.58 78.88) (width 0.6) (layer "B.Cu") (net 1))
 (segment (start 129.125 80.35) (end 130.6825 81.9075) (width 0.6) (layer "B.Cu") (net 1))
 (segment (start 161.67 74) (end 161.66 74.01) (width 0.6) (layer "B.Cu") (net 1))
 (segment (start 132.75 87.4) (end 132.75 83.975) (width 0.6) (layer "B.Cu") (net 1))
 (segment (start 140.67 78.93) (end 138.63 78.93) (width 0.6) (layer "B.Cu") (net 1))
 (segment (start 138.57 87.615) (end 139.915 88.96) (width 0.6) (layer "B.Cu") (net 11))
 (segment (start 145.03 83.59) (end 144.98 83.54) (width 0.6) (layer "B.Cu") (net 11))
 (segment (start 139.915 88.96) (end 145.03 88.96) (width 0.6) (layer "B.Cu") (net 11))
 (segment (start 145.03 88.96) (end 145.03 83.59) (width 0.6) (layer "B.Cu") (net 11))
 (segment (start 126.355 82.925) (end 125.02 81.59) (width 0.6) (layer "B.Cu") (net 2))
 (segment (start 126.355 85.35) (end 126.355 82.925) (width 0.6) (layer "B.Cu") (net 2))
 (segment (start 125.02 81.59) (end 125.02 76.46) (width 0.6) (layer "B.Cu") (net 2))
 (segment (start 126.035 75.445) (end 127.565 75.445) (width 0.6) (layer "B.Cu") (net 2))
 (segment (start 125.02 76.46) (end 126.035 75.445) (width 0.6) (layer "B.Cu") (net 2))
 (segment (start 136.915 62.4) (end 136.915 58.375) (width 0.6) (layer "B.Cu") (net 4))
 (segment (start 123.82 82.815) (end 123.855 82.85) (width 0.6) (layer "B.Cu") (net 4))
 (segment (start 136.825 62.31) (end 136.915 62.4) (width 0.6) (layer "B.Cu") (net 4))
 (segment (start 127.75 66.16) (end 131.6 62.31) (width 0.6) (layer "B.Cu") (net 4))
 (segment (start 123.82 68.09) (end 125.75 66.16) (width 0.6) (layer "B.Cu") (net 4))
 (segment (start 145.02 57.4) (end 148.69 61.07) (width 0.6) (layer "B.Cu") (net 4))
 (segment (start 136.915 58.375) (end 137.89 57.4) (width 0.6) (layer "B.Cu") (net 4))
 (segment (start 137.89 57.4) (end 145.02 57.4) (width 0.6) (layer "B.Cu") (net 4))
 (segment (start 125.75 66.16) (end 127.75 66.16) (width 0.6) (layer "B.Cu") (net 4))
 (segment (start 131.6 62.31) (end 136.825 62.31) (width 0.6) (layer "B.Cu") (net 4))
 (segment (start 123.82 68.09) (end 123.82 82.815) (width 0.6) (layer "B.Cu") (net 4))
 (segment (start 136.57 75.9) (end 137.08 76.41) (width 0.6) (layer "B.Cu") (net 6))
 (segment (start 137.08 76.41) (end 138.51 76.41) (width 0.6) (layer "B.Cu") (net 6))
 (segment (start 139.415 66.855) (end 136.57 69.7) (width 0.6) (layer "B.Cu") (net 6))
 (segment (start 138.51 76.41) (end 138.58 76.34) (width 0.6) (layer "B.Cu") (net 6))
 (segment (start 136.57 69.7) (end 136.57 75.9) (width 0.6) (layer "B.Cu") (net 6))
 (segment (start 139.415 66.855) (end 139.415 59.9) (width 0.6) (layer "B.Cu") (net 6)))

